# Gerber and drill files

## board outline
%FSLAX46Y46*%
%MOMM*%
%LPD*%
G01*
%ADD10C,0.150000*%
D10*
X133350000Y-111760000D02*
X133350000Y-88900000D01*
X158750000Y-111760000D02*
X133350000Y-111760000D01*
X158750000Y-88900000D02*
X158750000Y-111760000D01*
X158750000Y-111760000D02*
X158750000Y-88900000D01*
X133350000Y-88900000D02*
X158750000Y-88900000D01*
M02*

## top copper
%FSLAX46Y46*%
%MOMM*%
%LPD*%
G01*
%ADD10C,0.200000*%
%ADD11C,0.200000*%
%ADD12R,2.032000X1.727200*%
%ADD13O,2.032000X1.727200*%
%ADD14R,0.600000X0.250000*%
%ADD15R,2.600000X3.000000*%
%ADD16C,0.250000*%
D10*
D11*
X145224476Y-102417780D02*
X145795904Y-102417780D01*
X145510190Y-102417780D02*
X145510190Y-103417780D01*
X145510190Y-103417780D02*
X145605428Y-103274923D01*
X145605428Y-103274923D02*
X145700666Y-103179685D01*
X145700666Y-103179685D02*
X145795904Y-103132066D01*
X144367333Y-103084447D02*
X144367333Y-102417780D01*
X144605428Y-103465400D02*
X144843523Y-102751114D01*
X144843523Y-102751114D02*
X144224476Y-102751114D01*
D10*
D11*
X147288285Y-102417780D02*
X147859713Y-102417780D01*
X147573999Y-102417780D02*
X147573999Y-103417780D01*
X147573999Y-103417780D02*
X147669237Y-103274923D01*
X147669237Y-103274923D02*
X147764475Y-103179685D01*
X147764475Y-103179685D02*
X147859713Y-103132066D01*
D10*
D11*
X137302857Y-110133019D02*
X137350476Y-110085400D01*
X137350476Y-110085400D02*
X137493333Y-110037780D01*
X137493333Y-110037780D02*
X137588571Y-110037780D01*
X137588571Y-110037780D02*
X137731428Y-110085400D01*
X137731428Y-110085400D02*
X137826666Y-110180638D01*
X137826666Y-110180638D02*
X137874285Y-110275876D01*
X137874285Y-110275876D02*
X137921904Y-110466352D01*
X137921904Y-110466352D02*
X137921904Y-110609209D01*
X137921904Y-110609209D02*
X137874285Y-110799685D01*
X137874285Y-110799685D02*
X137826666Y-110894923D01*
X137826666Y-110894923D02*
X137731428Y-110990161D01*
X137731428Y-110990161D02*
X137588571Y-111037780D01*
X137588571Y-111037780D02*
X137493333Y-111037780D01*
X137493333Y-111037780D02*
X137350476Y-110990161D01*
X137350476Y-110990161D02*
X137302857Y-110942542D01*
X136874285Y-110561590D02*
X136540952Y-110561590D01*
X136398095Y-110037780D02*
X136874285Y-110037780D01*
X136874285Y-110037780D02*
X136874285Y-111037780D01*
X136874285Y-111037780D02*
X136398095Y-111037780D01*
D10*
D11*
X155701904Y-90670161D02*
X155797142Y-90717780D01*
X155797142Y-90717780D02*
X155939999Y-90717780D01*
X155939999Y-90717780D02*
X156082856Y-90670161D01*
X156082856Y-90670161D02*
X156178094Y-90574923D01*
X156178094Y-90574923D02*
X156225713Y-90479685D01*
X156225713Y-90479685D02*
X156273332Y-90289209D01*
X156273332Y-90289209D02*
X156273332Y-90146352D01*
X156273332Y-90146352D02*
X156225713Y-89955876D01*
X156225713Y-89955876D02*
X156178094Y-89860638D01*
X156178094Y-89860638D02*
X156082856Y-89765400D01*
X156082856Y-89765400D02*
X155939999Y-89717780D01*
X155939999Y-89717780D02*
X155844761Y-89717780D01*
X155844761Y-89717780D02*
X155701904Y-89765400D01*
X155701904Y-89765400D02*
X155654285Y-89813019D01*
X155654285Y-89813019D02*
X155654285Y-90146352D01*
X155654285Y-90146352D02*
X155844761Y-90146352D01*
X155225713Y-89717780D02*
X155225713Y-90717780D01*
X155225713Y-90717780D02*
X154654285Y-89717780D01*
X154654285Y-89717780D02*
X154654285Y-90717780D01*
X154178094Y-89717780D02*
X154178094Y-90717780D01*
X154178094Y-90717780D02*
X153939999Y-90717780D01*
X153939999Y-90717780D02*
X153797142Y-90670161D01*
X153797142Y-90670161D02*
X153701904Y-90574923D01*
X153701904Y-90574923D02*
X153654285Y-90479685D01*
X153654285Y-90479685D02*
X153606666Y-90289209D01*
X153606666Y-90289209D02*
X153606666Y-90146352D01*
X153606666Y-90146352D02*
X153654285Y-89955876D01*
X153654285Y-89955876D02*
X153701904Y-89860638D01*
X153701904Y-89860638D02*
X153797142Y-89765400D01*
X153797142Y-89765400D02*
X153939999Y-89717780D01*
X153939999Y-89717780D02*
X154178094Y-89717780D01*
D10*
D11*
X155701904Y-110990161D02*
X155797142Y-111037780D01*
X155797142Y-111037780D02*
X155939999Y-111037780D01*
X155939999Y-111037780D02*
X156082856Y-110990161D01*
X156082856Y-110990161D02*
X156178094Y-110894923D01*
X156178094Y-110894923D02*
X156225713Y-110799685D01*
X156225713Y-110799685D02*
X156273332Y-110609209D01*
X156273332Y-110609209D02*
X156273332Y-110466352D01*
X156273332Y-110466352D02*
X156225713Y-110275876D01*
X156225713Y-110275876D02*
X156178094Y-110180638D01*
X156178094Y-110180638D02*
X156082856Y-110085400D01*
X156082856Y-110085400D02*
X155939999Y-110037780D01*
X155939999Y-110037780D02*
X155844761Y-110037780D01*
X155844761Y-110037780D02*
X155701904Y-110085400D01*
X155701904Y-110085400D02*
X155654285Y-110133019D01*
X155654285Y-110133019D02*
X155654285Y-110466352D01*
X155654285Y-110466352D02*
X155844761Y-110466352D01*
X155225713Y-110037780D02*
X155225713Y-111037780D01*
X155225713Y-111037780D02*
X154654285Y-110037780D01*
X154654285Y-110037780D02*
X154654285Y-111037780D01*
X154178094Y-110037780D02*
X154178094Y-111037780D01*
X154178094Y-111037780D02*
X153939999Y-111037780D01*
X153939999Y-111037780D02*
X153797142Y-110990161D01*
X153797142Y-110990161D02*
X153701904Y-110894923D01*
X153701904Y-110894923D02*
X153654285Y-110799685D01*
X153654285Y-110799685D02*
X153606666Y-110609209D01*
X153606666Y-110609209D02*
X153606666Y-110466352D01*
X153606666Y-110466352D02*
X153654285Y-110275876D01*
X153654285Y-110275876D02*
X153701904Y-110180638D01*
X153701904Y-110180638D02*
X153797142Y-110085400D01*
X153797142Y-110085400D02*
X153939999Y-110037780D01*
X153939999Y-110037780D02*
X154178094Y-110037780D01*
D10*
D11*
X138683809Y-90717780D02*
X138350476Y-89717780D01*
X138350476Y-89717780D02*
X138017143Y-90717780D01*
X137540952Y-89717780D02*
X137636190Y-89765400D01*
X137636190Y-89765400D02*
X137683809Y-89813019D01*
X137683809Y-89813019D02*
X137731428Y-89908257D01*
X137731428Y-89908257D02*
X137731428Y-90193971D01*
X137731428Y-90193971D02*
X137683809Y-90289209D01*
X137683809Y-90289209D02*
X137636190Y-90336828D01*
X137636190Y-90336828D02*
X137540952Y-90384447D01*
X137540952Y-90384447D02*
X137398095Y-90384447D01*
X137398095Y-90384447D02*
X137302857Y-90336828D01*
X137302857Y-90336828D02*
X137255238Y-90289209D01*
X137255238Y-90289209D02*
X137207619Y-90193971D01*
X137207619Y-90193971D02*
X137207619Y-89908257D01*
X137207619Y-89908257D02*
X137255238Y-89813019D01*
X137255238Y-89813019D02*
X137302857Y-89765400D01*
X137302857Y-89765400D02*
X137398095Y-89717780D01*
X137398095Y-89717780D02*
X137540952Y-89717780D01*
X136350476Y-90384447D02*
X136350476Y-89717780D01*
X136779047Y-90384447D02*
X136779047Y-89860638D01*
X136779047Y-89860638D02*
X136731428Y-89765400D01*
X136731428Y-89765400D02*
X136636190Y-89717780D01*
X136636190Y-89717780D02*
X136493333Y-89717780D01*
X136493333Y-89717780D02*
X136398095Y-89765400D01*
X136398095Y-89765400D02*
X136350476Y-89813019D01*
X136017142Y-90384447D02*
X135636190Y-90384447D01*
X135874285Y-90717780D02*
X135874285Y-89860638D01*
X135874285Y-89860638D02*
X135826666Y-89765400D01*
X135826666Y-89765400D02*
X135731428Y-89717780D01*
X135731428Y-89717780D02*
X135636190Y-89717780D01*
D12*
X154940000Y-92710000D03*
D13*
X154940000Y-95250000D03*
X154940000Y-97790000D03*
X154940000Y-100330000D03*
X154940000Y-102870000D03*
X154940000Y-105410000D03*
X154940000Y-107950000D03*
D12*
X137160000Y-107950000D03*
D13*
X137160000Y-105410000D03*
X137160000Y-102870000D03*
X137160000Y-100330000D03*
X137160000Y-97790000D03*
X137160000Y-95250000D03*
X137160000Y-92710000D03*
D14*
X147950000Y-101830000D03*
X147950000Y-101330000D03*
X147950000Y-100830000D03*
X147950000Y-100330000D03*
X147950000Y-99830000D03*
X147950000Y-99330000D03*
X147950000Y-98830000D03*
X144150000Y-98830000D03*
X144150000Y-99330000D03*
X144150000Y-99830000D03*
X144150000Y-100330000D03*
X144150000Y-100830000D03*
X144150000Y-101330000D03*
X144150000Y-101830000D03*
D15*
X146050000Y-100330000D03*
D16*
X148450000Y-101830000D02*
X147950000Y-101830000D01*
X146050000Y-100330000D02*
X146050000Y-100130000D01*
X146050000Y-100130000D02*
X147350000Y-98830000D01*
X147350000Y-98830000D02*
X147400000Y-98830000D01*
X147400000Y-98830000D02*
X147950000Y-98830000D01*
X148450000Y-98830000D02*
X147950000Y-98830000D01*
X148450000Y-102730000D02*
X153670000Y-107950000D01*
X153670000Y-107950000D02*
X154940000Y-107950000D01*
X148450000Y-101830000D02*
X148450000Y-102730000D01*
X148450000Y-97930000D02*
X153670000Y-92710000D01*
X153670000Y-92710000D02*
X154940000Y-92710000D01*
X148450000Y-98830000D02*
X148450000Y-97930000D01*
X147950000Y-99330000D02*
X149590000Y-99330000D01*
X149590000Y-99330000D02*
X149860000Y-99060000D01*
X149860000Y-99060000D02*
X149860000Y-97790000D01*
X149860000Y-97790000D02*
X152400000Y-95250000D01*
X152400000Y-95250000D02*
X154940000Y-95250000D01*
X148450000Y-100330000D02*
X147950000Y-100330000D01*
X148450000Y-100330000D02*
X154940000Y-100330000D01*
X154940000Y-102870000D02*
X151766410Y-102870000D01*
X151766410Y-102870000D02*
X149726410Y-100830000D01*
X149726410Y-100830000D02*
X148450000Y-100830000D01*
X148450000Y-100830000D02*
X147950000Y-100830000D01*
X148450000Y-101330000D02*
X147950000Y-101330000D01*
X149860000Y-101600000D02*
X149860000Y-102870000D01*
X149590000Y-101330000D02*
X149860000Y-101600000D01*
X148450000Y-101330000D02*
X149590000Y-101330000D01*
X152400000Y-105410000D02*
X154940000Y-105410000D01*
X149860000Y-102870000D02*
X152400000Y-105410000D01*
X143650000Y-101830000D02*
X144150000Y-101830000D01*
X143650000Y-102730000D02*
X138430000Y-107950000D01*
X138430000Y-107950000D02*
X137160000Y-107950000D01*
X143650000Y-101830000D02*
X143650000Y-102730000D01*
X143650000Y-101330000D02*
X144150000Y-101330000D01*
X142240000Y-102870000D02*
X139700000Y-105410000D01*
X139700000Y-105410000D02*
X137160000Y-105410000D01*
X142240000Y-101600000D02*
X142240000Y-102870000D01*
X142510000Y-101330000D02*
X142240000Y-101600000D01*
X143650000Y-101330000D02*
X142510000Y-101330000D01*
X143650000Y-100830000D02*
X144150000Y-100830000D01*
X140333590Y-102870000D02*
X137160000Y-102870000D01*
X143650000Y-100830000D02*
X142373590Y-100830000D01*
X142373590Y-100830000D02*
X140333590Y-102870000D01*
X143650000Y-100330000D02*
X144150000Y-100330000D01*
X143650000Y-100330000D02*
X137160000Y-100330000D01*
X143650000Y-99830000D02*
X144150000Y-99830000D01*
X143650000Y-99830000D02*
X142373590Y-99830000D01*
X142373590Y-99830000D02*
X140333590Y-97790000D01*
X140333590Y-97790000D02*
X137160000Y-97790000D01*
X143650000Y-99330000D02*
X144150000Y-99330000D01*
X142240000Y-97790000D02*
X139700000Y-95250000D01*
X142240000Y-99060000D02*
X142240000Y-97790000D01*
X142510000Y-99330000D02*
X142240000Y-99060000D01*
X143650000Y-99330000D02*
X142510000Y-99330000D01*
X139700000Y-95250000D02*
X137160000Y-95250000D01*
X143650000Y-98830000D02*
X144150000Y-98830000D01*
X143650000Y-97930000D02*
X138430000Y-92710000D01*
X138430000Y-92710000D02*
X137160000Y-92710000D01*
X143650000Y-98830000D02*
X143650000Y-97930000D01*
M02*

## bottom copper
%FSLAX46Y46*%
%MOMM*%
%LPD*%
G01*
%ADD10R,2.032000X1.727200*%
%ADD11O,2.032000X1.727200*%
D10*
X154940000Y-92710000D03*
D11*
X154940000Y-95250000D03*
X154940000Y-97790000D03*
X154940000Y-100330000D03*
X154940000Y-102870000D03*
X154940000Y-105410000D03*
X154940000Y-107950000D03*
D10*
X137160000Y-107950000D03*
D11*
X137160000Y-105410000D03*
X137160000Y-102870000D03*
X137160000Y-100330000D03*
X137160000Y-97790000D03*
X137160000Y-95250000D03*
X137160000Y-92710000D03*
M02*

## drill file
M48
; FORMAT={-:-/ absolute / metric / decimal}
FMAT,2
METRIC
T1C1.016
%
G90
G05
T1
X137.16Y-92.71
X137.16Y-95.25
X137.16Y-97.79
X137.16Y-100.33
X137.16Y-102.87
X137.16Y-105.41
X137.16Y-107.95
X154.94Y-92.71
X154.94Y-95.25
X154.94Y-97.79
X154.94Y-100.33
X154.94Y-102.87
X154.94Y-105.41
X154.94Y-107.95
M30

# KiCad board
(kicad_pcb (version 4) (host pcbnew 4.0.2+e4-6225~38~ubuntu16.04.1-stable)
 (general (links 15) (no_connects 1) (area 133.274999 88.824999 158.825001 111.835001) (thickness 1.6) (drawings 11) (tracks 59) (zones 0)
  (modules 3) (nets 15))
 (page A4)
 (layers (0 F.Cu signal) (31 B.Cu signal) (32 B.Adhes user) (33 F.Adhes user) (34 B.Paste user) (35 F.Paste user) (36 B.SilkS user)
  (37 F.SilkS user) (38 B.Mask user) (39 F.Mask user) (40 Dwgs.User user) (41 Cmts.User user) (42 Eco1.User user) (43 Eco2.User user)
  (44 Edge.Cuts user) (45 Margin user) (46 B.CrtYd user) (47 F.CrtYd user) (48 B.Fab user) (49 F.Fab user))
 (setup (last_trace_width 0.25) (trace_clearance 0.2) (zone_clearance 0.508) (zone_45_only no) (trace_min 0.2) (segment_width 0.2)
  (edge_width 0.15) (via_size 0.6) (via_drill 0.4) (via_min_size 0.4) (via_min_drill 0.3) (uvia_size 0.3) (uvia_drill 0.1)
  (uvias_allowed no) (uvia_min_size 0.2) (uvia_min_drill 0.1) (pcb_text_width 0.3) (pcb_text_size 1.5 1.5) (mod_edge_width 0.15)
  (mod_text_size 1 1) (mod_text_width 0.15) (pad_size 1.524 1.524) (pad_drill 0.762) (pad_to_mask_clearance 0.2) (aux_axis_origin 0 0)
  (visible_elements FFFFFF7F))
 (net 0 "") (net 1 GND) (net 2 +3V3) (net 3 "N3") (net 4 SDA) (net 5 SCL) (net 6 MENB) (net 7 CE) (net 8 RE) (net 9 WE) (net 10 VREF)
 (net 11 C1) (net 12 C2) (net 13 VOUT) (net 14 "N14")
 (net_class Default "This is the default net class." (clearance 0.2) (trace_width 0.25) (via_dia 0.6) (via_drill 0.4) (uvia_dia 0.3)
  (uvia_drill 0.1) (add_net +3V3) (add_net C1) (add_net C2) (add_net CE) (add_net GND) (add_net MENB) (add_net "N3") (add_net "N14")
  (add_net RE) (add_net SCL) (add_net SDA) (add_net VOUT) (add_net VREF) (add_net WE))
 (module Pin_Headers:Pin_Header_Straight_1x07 (layer F.Cu) (at 154.94 92.71)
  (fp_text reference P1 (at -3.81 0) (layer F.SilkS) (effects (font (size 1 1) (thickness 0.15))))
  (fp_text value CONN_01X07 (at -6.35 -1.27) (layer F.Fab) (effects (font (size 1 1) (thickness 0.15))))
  (pad 1 thru_hole rect (at 0 0) (size 2.032 1.7272) (drill 1.016) (layers *.Cu *.Mask F.SilkS) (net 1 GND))
  (pad 2 thru_hole oval (at 0 2.54) (size 2.032 1.7272) (drill 1.016) (layers *.Cu *.Mask F.SilkS) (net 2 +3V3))
  (pad 3 thru_hole oval (at 0 5.08) (size 2.032 1.7272) (drill 1.016) (layers *.Cu *.Mask F.SilkS) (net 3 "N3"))
  (pad 4 thru_hole oval (at 0 7.62) (size 2.032 1.7272) (drill 1.016) (layers *.Cu *.Mask F.SilkS) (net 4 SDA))
  (pad 5 thru_hole oval (at 0 10.16) (size 2.032 1.7272) (drill 1.016) (layers *.Cu *.Mask F.SilkS) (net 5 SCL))
  (pad 6 thru_hole oval (at 0 12.7) (size 2.032 1.7272) (drill 1.016) (layers *.Cu *.Mask F.SilkS) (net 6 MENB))
  (pad 7 thru_hole oval (at 0 15.24) (size 2.032 1.7272) (drill 1.016) (layers *.Cu *.Mask F.SilkS) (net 1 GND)))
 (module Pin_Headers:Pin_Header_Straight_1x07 (layer F.Cu) (at 137.16 107.95 180)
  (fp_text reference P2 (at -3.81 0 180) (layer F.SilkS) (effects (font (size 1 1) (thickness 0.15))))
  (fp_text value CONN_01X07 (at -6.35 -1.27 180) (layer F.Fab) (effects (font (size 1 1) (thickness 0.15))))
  (pad 1 thru_hole rect (at 0 0 180) (size 2.032 1.7272) (drill 1.016) (layers *.Cu *.Mask F.SilkS) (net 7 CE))
  (pad 2 thru_hole oval (at 0 2.54 180) (size 2.032 1.7272) (drill 1.016) (layers *.Cu *.Mask F.SilkS) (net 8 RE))
  (pad 3 thru_hole oval (at 0 5.08 180) (size 2.032 1.7272) (drill 1.016) (layers *.Cu *.Mask F.SilkS) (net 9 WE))
  (pad 4 thru_hole oval (at 0 7.62 180) (size 2.032 1.7272) (drill 1.016) (layers *.Cu *.Mask F.SilkS) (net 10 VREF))
  (pad 5 thru_hole oval (at 0 10.16 180) (size 2.032 1.7272) (drill 1.016) (layers *.Cu *.Mask F.SilkS) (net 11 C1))
  (pad 6 thru_hole oval (at 0 12.7 180) (size 2.032 1.7272) (drill 1.016) (layers *.Cu *.Mask F.SilkS) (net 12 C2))
  (pad 7 thru_hole oval (at 0 15.24 180) (size 2.032 1.7272) (drill 1.016) (layers *.Cu *.Mask F.SilkS) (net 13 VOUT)))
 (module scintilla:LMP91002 (layer F.Cu) (at 146.05 100.33 90)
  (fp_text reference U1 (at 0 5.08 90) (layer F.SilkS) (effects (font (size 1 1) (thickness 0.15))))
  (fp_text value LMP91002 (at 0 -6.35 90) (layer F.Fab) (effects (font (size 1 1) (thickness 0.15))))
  (pad 1 smd rect (at -1.5 1.9 90) (size 0.25 0.6) (layers F.Cu F.Paste F.Mask) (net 1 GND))
  (pad 2 smd rect (at -1 1.9 90) (size 0.25 0.6) (layers F.Cu F.Paste F.Mask) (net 6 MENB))
  (pad 3 smd rect (at -0.5 1.9 90) (size 0.25 0.6) (layers F.Cu F.Paste F.Mask) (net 5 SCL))
  (pad 4 smd rect (at 0 1.9 90) (size 0.25 0.6) (layers F.Cu F.Paste F.Mask) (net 4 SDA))
  (pad 5 smd rect (at 0.5 1.9 90) (size 0.25 0.6) (layers F.Cu F.Paste F.Mask) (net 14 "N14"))
  (pad 6 smd rect (at 1 1.9 90) (size 0.25 0.6) (layers F.Cu F.Paste F.Mask) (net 2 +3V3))
  (pad 7 smd rect (at 1.5 1.9 90) (size 0.25 0.6) (layers F.Cu F.Paste F.Mask) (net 1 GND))
  (pad 8 smd rect (at 1.5 -1.9 90) (size 0.25 0.6) (layers F.Cu F.Paste F.Mask) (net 13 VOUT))
  (pad 9 smd rect (at 1 -1.9 90) (size 0.25 0.6) (layers F.Cu F.Paste F.Mask) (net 12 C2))
  (pad 10 smd rect (at 0.5 -1.9 90) (size 0.25 0.6) (layers F.Cu F.Paste F.Mask) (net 11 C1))
  (pad 11 smd rect (at 0 -1.9 90) (size 0.25 0.6) (layers F.Cu F.Paste F.Mask) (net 10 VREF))
  (pad 12 smd rect (at -0.5 -1.9 90) (size 0.25 0.6) (layers F.Cu F.Paste F.Mask) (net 9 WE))
  (pad 13 smd rect (at -1 -1.9 90) (size 0.25 0.6) (layers F.Cu F.Paste F.Mask) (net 8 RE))
  (pad 14 smd rect (at -1.5 -1.9 90) (size 0.25 0.6) (layers F.Cu F.Paste F.Mask) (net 7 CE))
  (pad 15 smd rect (at 0 0 90) (size 3 2.6) (layers F.Cu F.Paste F.Mask) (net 1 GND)))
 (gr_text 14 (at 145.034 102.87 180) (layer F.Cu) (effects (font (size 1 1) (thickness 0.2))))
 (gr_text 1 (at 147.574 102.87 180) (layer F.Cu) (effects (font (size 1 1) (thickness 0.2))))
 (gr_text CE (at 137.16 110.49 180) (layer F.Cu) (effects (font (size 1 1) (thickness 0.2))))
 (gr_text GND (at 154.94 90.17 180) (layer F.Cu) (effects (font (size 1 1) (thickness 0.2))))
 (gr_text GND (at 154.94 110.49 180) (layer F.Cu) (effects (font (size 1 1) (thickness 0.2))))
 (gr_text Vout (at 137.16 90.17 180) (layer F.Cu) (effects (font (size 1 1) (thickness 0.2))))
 (gr_line (start 133.35 111.76) (end 133.35 88.9) (layer Edge.Cuts) (width 0.15))
 (gr_line (start 158.75 111.76) (end 133.35 111.76) (layer Edge.Cuts) (width 0.15))
 (gr_line (start 158.75 88.9) (end 158.75 111.76) (layer Edge.Cuts) (width 0.15))
 (gr_line (start 158.75 111.76) (end 158.75 88.9) (layer Edge.Cuts) (width 0.15))
 (gr_line (start 133.35 88.9) (end 158.75 88.9) (layer Edge.Cuts) (width 0.15))
 (segment (start 148.45 101.83) (end 147.95 101.83) (width 0.25) (layer F.Cu) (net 1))
 (segment (start 146.05 100.33) (end 146.05 100.13) (width 0.25) (layer F.Cu) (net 1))
 (segment (start 146.05 100.13) (end 147.35 98.83) (width 0.25) (layer F.Cu) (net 1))
 (segment (start 147.35 98.83) (end 147.4 98.83) (width 0.25) (layer F.Cu) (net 1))
 (segment (start 147.4 98.83) (end 147.95 98.83) (width 0.25) (layer F.Cu) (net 1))
 (segment (start 148.45 98.83) (end 147.95 98.83) (width 0.25) (layer F.Cu) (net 1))
 (segment (start 148.45 102.73) (end 153.67 107.95) (width 0.25) (layer F.Cu) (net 1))
 (segment (start 153.67 107.95) (end 154.94 107.95) (width 0.25) (layer F.Cu) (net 1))
 (segment (start 148.45 101.83) (end 148.45 102.73) (width 0.25) (layer F.Cu) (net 1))
 (segment (start 148.45 97.93) (end 153.67 92.71) (width 0.25) (layer F.Cu) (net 1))
 (segment (start 153.67 92.71) (end 154.94 92.71) (width 0.25) (layer F.Cu) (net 1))
 (segment (start 148.45 98.83) (end 148.45 97.93) (width 0.25) (layer F.Cu) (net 1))
 (segment (start 147.95 99.33) (end 149.59 99.33) (width 0.25) (layer F.Cu) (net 2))
 (segment (start 149.59 99.33) (end 149.86 99.06) (width 0.25) (layer F.Cu) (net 2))
 (segment (start 149.86 99.06) (end 149.86 97.79) (width 0.25) (layer F.Cu) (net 2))
 (segment (start 149.86 97.79) (end 152.4 95.25) (width 0.25) (layer F.Cu) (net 2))
 (segment (start 152.4 95.25) (end 154.94 95.25) (width 0.25) (layer F.Cu) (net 2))
 (segment (start 148.45 100.33) (end 147.95 100.33) (width 0.25) (layer F.Cu) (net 4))
 (segment (start 148.45 100.33) (end 154.94 100.33) (width 0.25) (layer F.Cu) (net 4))
 (segment (start 154.94 102.87) (end 151.76641 102.87) (width 0.25) (layer F.Cu) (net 5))
 (segment (start 151.76641 102.87) (end 149.72641 100.83) (width 0.25) (layer F.Cu) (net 5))
 (segment (start 149.72641 100.83) (end 148.45 100.83) (width 0.25) (layer F.Cu) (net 5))
 (segment (start 148.45 100.83) (end 147.95 100.83) (width 0.25) (layer F.Cu) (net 5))
 (segment (start 148.45 101.33) (end 147.95 101.33) (width 0.25) (layer F.Cu) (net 6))
 (segment (start 149.86 101.6) (end 149.86 102.87) (width 0.25) (layer F.Cu) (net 6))
 (segment (start 149.59 101.33) (end 149.86 101.6) (width 0.25) (layer F.Cu) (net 6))
 (segment (start 148.45 101.33) (end 149.59 101.33) (width 0.25) (layer F.Cu) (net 6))
 (segment (start 152.4 105.41) (end 154.94 105.41) (width 0.25) (layer F.Cu) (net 6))
 (segment (start 149.86 102.87) (end 152.4 105.41) (width 0.25) (layer F.Cu) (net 6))
 (segment (start 143.65 101.83) (end 144.15 101.83) (width 0.25) (layer F.Cu) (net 7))
 (segment (start 143.65 102.73) (end 138.43 107.95) (width 0.25) (layer F.Cu) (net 7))
 (segment (start 138.43 107.95) (end 137.16 107.95) (width 0.25) (layer F.Cu) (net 7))
 (segment (start 143.65 101.83) (end 143.65 102.73) (width 0.25) (layer F.Cu) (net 7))
 (segment (start 143.65 101.33) (end 144.15 101.33) (width 0.25) (layer F.Cu) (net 8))
 (segment (start 142.24 102.87) (end 139.7 105.41) (width 0.25) (layer F.Cu) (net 8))
 (segment (start 139.7 105.41) (end 137.16 105.41) (width 0.25) (layer F.Cu) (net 8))
 (segment (start 142.24 101.6) (end 142.24 102.87) (width 0.25) (layer F.Cu) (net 8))
 (segment (start 142.51 101.33) (end 142.24 101.6) (width 0.25) (layer F.Cu) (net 8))
 (segment (start 143.65 101.33) (end 142.51 101.33) (width 0.25) (layer F.Cu) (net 8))
 (segment (start 143.65 100.83) (end 144.15 100.83) (width 0.25) (layer F.Cu) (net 9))
 (segment (start 140.33359 102.87) (end 137.16 102.87) (width 0.25) (layer F.Cu) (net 9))
 (segment (start 143.65 100.83) (end 142.37359 100.83) (width 0.25) (layer F.Cu) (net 9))
 (segment (start 142.37359 100.83) (end 140.33359 102.87) (width 0.25) (layer F.Cu) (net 9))
 (segment (start 143.65 100.33) (end 144.15 100.33) (width 0.25) (layer F.Cu) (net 10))
 (segment (start 143.65 100.33) (end 137.16 100.33) (width 0.25) (layer F.Cu) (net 10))
 (segment (start 143.65 99.83) (end 144.15 99.83) (width 0.25) (layer F.Cu) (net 11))
 (segment (start 143.65 99.83) (end 142.37359 99.83) (width 0.25) (layer F.Cu) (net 11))
 (segment (start 142.37359 99.83) (end 140.33359 97.79) (width 0.25) (layer F.Cu) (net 11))
 (segment (start 140.33359 97.79) (end 137.16 97.79) (width 0.25) (layer F.Cu) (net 11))
 (segment (start 143.65 99.33) (end 144.15 99.33) (width 0.25) (layer F.Cu) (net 12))
 (segment (start 142.24 97.79) (end 139.7 95.25) (width 0.25) (layer F.Cu) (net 12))
 (segment (start 142.24 99.06) (end 142.24 97.79) (width 0.25) (layer F.Cu) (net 12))
 (segment (start 142.51 99.33) (end 142.24 99.06) (width 0.25) (layer F.Cu) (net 12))
 (segment (start 143.65 99.33) (end 142.51 99.33) (width 0.25) (layer F.Cu) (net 12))
 (segment (start 139.7 95.25) (end 137.16 95.25) (width 0.25) (layer F.Cu) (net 12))
 (segment (start 143.65 98.83) (end 144.15 98.83) (width 0.25) (layer F.Cu) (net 13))
 (segment (start 143.65 97.93) (end 138.43 92.71) (width 0.25) (layer F.Cu) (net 13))
 (segment (start 138.43 92.71) (end 137.16 92.71) (width 0.25) (layer F.Cu) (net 13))
 (segment (start 143.65 98.83) (end 143.65 97.93) (width 0.25) (layer F.Cu) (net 13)))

